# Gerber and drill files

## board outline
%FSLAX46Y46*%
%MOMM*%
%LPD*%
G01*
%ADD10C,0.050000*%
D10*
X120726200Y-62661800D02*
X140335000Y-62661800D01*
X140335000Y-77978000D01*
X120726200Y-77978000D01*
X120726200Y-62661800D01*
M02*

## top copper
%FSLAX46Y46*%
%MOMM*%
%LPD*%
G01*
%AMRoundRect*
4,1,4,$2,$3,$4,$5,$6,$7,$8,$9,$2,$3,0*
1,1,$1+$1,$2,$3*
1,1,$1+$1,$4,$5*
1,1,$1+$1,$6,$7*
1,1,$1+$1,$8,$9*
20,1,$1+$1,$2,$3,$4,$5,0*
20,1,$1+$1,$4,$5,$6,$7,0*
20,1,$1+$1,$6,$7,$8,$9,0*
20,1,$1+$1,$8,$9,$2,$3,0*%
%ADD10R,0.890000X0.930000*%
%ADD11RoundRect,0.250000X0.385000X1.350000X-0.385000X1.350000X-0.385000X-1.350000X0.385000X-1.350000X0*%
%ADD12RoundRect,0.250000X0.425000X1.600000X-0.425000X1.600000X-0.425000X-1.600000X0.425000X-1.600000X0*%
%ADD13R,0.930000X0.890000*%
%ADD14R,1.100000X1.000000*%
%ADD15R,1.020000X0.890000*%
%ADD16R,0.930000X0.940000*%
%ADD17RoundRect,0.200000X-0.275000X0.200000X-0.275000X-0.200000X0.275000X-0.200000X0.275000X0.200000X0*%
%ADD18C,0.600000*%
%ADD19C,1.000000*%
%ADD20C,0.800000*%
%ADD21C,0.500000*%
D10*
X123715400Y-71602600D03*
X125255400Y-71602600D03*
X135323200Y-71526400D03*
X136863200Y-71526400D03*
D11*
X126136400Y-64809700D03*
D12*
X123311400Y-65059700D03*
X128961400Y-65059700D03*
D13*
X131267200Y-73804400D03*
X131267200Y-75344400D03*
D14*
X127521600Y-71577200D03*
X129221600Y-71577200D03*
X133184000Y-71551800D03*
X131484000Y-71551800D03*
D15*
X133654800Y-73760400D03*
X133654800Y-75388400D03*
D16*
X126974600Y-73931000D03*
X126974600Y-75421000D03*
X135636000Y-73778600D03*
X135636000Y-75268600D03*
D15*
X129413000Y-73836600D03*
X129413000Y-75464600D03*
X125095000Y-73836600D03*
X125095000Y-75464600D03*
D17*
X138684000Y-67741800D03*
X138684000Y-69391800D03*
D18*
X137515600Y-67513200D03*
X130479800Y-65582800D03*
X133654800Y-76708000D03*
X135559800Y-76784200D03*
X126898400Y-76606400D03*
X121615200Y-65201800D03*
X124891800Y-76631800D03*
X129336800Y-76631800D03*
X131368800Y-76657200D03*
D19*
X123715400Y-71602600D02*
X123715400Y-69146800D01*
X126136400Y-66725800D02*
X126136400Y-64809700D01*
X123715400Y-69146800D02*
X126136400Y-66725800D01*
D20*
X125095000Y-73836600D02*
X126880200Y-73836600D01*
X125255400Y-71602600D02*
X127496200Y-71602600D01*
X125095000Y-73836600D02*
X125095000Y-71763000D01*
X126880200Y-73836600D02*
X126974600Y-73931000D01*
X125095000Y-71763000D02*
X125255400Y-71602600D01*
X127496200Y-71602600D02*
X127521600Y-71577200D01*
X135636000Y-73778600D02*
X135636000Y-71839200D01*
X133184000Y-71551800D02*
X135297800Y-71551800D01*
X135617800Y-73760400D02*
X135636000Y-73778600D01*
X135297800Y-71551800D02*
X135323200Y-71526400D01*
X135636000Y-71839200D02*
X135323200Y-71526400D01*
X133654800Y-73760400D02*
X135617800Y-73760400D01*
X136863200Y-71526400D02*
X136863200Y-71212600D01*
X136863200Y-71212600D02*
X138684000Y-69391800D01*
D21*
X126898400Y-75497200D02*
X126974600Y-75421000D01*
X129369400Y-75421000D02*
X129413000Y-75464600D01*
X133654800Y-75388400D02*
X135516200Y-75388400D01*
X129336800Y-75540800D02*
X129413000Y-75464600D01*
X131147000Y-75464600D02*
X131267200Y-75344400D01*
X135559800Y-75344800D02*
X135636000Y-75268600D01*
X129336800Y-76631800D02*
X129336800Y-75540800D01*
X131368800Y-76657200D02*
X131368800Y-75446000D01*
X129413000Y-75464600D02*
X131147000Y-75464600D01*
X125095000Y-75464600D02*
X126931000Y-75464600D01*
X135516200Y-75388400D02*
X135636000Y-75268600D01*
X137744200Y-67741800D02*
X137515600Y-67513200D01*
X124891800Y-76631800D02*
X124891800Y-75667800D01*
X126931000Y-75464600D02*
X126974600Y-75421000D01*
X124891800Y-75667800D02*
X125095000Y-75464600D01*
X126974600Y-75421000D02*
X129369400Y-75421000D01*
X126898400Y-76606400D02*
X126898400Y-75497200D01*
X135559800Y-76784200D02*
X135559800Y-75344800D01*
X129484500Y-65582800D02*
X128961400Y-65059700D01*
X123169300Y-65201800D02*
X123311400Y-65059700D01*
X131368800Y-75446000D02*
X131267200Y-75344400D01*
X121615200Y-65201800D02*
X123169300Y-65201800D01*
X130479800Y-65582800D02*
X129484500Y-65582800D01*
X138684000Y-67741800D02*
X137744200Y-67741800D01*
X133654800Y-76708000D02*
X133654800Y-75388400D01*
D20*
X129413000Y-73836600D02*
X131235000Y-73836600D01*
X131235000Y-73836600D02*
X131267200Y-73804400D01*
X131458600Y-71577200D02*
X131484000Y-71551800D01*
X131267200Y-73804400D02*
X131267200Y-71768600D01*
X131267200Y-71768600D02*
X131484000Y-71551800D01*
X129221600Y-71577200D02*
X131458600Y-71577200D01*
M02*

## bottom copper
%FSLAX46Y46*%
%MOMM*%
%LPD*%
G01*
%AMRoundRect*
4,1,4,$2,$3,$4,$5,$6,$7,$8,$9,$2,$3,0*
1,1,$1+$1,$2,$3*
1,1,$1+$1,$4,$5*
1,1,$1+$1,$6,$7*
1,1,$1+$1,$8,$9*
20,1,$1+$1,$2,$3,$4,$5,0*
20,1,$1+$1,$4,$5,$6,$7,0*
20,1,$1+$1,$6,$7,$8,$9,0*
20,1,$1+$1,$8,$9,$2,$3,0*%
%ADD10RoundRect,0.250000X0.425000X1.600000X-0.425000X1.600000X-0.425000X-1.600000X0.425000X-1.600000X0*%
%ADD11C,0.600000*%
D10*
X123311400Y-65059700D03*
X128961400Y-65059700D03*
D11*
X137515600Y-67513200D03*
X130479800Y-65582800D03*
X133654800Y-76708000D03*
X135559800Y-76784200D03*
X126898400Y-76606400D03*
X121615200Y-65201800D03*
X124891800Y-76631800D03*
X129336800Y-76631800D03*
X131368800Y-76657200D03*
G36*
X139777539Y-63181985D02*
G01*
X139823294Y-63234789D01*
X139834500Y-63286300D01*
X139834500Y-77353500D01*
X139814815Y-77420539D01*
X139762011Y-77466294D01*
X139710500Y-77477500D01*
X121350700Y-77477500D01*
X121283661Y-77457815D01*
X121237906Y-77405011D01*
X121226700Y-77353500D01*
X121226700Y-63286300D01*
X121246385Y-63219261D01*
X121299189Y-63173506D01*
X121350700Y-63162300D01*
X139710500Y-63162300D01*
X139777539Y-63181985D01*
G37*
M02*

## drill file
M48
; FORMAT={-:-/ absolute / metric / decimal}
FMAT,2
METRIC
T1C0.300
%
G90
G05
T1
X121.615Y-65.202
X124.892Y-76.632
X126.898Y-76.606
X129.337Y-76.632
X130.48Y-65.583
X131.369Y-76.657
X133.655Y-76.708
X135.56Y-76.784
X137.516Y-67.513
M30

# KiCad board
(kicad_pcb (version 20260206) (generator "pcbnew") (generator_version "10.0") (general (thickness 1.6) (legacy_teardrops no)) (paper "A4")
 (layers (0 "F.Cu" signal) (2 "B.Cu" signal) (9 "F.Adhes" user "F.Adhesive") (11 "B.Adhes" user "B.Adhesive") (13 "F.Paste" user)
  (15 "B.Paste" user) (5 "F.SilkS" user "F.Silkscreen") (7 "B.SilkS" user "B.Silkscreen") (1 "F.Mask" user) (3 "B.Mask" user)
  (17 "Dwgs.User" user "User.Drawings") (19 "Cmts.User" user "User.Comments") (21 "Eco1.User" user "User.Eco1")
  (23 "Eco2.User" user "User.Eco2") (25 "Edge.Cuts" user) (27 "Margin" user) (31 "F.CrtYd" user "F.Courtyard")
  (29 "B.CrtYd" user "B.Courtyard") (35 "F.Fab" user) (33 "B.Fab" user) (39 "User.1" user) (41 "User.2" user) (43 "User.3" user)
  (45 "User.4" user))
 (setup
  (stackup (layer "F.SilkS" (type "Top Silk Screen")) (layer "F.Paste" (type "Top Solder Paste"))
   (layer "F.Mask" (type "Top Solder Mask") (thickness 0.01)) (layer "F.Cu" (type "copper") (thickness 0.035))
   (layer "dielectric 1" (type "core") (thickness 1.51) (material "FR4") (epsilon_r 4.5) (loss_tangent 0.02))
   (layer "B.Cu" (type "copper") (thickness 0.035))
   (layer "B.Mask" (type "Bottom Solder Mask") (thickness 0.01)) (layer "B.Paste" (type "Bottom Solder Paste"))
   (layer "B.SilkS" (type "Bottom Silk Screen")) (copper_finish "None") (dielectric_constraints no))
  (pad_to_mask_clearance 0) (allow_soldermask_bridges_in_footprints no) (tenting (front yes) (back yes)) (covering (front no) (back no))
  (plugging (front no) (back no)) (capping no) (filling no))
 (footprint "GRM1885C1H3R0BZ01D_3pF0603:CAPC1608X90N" (layer "F.Cu") (at 124.4854 71.6026)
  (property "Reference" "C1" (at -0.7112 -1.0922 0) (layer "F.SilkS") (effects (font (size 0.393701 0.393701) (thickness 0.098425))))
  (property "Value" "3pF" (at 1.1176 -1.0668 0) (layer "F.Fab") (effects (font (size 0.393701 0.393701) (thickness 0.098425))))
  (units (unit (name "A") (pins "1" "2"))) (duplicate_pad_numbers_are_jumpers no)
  (pad "1" smd rect (at -0.77 0) (size 0.89 0.93) (layers "F.Cu" "F.Mask" "F.Paste") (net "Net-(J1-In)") (solder_mask_margin 0.102))
  (pad "2" smd rect (at 0.77 0) (size 0.89 0.93) (layers "F.Cu" "F.Mask" "F.Paste") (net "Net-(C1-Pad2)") (solder_mask_margin 0.102)))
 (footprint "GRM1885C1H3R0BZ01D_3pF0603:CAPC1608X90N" (layer "F.Cu") (at 136.0932 71.5264)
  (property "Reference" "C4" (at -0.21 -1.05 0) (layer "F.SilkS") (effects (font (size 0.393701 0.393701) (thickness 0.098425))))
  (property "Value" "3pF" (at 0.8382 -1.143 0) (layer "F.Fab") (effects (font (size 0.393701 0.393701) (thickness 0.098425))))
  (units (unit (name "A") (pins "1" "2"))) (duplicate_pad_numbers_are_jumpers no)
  (pad "1" smd rect (at -0.77 0) (size 0.89 0.93) (layers "F.Cu" "F.Mask" "F.Paste") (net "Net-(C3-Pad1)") (solder_mask_margin 0.102))
  (pad "2" smd rect (at 0.77 0) (size 0.89 0.93) (layers "F.Cu" "F.Mask" "F.Paste") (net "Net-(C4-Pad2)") (solder_mask_margin 0.102)))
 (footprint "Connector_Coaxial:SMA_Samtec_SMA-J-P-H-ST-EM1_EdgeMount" (layer "F.Cu") (at 126.1364 64.8097 90)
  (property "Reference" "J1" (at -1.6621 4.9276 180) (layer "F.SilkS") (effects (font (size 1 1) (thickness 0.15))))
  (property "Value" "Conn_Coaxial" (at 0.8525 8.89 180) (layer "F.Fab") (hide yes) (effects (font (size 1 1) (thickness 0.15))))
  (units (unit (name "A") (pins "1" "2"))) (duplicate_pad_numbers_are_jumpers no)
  (pad "1" smd roundrect (at 0 0 180) (size 1.27 3.2) (layers "F.Cu" "F.Mask") (roundrect_rratio 0.1968503937) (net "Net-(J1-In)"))
  (pad "2" smd roundrect (at -0.25 -2.825 180) (size 1.35 3.7) (layers "F.Cu" "F.Mask") (roundrect_rratio 0.1851851852) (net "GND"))
  (pad "2" smd roundrect (at -0.25 -2.825 180) (size 1.35 3.7) (layers "B.Cu" "B.Mask") (roundrect_rratio 0.1851851852) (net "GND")
   (zone_connect 2))
  (pad "2" smd roundrect (at -0.25 2.825 180) (size 1.35 3.7) (layers "F.Cu" "F.Mask") (roundrect_rratio 0.1851851852) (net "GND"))
  (pad "2" smd roundrect (at -0.25 2.825 180) (size 1.35 3.7) (layers "B.Cu" "B.Mask") (roundrect_rratio 0.1851851852) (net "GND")
   (zone_connect 2)))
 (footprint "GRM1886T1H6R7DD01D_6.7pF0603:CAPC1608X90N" (layer "F.Cu") (at 131.2672 74.5744 -90)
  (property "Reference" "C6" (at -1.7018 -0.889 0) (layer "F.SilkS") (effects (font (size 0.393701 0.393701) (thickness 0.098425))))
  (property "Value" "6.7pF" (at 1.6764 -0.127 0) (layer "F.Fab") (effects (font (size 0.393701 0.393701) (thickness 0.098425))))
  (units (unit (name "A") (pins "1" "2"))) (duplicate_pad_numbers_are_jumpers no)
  (pad "1" smd rect (at -0.77 0 270) (size 0.89 0.93) (layers "F.Cu" "F.Mask" "F.Paste") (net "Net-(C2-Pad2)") (solder_mask_margin 0.102))
  (pad "2" smd rect (at 0.77 0 270) (size 0.89 0.93) (layers "F.Cu" "F.Mask" "F.Paste") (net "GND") (solder_mask_margin 0.102)))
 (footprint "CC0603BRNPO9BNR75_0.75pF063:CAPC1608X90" (layer "F.Cu") (at 128.3716 71.5772)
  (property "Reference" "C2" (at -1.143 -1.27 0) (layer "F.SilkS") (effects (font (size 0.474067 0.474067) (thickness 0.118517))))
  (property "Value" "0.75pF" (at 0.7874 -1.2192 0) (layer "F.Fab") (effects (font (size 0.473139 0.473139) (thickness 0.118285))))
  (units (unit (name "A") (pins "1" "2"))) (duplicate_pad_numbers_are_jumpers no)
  (pad "1" smd rect (at -0.85 0) (size 1.1 1) (layers "F.Cu" "F.Mask" "F.Paste") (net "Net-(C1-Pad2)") (solder_mask_margin 0.102))
  (pad "2" smd rect (at 0.85 0) (size 1.1 1) (layers "F.Cu" "F.Mask" "F.Paste") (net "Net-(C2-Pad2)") (solder_mask_margin 0.102)))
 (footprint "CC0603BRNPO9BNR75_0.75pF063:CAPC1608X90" (layer "F.Cu") (at 132.334 71.5518 180)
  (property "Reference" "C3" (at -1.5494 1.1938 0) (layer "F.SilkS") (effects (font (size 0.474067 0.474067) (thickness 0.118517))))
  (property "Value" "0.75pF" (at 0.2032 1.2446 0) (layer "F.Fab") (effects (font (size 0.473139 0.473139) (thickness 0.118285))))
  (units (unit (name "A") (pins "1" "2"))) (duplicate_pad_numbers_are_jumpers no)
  (pad "1" smd rect (at -0.85 0 180) (size 1.1 1) (layers "F.Cu" "F.Mask" "F.Paste") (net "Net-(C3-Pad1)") (solder_mask_margin 0.102))
  (pad "2" smd rect (at 0.85 0 180) (size 1.1 1) (layers "F.Cu" "F.Mask" "F.Paste") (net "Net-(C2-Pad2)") (solder_mask_margin 0.102)))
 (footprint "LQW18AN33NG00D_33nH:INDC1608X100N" (layer "F.Cu") (at 133.6548 74.5744 -90)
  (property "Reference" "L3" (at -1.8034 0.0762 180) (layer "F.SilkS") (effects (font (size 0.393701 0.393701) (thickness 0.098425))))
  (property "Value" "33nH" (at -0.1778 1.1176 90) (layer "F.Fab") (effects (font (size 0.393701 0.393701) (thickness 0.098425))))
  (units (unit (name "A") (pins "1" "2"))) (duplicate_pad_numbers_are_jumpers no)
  (pad "1" smd rect (at -0.814 0 270) (size 0.89 1.02) (layers "F.Cu" "F.Mask" "F.Paste") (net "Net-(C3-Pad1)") (solder_mask_margin 0.102))
  (pad "2" smd rect (at 0.814 0 270) (size 0.89 1.02) (layers "F.Cu" "F.Mask" "F.Paste") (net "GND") (solder_mask_margin 0.102)))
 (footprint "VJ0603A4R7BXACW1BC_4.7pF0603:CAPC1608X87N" (layer "F.Cu") (at 126.9746 74.676 -90)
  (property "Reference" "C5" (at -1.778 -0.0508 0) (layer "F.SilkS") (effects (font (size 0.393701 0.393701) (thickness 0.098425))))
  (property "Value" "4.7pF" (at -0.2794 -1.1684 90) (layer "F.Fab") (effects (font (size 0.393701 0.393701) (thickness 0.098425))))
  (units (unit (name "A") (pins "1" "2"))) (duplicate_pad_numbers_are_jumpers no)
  (pad "1" smd rect (at -0.745 0 270) (size 0.94 0.93) (layers "F.Cu" "F.Mask" "F.Paste") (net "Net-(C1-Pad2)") (solder_mask_margin 0.102))
  (pad "2" smd rect (at 0.745 0 270) (size 0.94 0.93) (layers "F.Cu" "F.Mask" "F.Paste") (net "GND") (solder_mask_margin 0.102)))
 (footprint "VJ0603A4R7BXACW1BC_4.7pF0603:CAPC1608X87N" (layer "F.Cu") (at 135.636 74.5236 -90)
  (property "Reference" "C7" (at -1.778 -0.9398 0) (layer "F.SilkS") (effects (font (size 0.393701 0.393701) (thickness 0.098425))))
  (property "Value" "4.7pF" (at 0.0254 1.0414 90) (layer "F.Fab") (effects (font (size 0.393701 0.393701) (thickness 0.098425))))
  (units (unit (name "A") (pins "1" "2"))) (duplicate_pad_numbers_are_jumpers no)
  (pad "1" smd rect (at -0.745 0 270) (size 0.94 0.93) (layers "F.Cu" "F.Mask" "F.Paste") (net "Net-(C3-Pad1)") (solder_mask_margin 0.102))
  (pad "2" smd rect (at 0.745 0 270) (size 0.94 0.93) (layers "F.Cu" "F.Mask" "F.Paste") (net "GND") (solder_mask_margin 0.102)))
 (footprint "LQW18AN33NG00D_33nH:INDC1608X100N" (layer "F.Cu") (at 129.413 74.6506 -90)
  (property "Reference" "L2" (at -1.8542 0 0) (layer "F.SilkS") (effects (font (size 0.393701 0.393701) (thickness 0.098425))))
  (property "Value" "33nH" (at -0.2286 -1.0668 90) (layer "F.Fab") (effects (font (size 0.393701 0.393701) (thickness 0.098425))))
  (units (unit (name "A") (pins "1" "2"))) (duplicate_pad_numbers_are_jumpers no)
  (pad "1" smd rect (at -0.814 0 270) (size 0.89 1.02) (layers "F.Cu" "F.Mask" "F.Paste") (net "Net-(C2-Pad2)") (solder_mask_margin 0.102))
  (pad "2" smd rect (at 0.814 0 270) (size 0.89 1.02) (layers "F.Cu" "F.Mask" "F.Paste") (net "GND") (solder_mask_margin 0.102)))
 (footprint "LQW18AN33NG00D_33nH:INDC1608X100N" (layer "F.Cu") (at 125.095 74.6506 -90)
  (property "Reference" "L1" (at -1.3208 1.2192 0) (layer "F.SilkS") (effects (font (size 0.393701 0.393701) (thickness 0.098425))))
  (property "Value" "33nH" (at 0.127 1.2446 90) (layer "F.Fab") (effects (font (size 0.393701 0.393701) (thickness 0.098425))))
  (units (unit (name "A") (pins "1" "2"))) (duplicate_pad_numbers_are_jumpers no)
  (pad "1" smd rect (at -0.814 0 270) (size 0.89 1.02) (layers "F.Cu" "F.Mask" "F.Paste") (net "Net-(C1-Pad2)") (solder_mask_margin 0.102))
  (pad "2" smd rect (at 0.814 0 270) (size 0.89 1.02) (layers "F.Cu" "F.Mask" "F.Paste") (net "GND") (solder_mask_margin 0.102)))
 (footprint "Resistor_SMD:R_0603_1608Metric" (layer "F.Cu") (at 138.684 68.5668 -90)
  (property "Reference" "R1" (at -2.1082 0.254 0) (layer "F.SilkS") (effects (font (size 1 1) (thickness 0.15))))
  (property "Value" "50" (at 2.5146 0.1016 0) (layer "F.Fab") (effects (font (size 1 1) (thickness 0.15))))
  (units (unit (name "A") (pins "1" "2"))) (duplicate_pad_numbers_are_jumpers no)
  (pad "1" smd roundrect (at -0.825 0 270) (size 0.8 0.95) (layers "F.Cu" "F.Mask" "F.Paste") (roundrect_rratio 0.25) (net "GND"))
  (pad "2" smd roundrect (at 0.825 0 270) (size 0.8 0.95) (layers "F.Cu" "F.Mask" "F.Paste") (roundrect_rratio 0.25) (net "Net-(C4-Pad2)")))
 (gr_rect (start 120.7262 62.6618) (end 140.335 77.978) (stroke (width 0.05) (type default)) (fill no) (layer "Edge.Cuts"))
 (segment (start 123.7154 71.6026) (end 123.7154 69.1468) (width 1) (layer "F.Cu") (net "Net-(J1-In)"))
 (segment (start 126.1364 66.7258) (end 126.1364 64.8097) (width 1) (layer "F.Cu") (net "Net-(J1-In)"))
 (segment (start 123.7154 69.1468) (end 126.1364 66.7258) (width 1) (layer "F.Cu") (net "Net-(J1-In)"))
 (segment (start 125.095 73.8366) (end 126.8802 73.8366) (width 0.8) (layer "F.Cu") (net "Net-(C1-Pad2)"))
 (segment (start 125.2554 71.6026) (end 127.4962 71.6026) (width 0.8) (layer "F.Cu") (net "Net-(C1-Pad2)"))
 (segment (start 125.095 73.8366) (end 125.095 71.763) (width 0.8) (layer "F.Cu") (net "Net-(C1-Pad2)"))
 (segment (start 126.8802 73.8366) (end 126.9746 73.931) (width 0.8) (layer "F.Cu") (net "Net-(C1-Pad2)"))
 (segment (start 125.095 71.763) (end 125.2554 71.6026) (width 0.8) (layer "F.Cu") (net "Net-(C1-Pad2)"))
 (segment (start 127.4962 71.6026) (end 127.5216 71.5772) (width 0.8) (layer "F.Cu") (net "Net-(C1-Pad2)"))
 (segment (start 135.636 73.7786) (end 135.636 71.8392) (width 0.8) (layer "F.Cu") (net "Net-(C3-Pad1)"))
 (segment (start 133.184 71.5518) (end 135.2978 71.5518) (width 0.8) (layer "F.Cu") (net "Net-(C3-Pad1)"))
 (segment (start 135.6178 73.7604) (end 135.636 73.7786) (width 0.8) (layer "F.Cu") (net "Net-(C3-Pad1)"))
 (segment (start 135.2978 71.5518) (end 135.3232 71.5264) (width 0.8) (layer "F.Cu") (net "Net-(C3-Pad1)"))
 (segment (start 135.636 71.8392) (end 135.3232 71.5264) (width 0.8) (layer "F.Cu") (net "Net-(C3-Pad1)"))
 (segment (start 133.6548 73.7604) (end 135.6178 73.7604) (width 0.8) (layer "F.Cu") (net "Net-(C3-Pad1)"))
 (segment (start 136.8632 71.5264) (end 136.8632 71.2126) (width 0.8) (layer "F.Cu") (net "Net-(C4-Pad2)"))
 (segment (start 136.8632 71.2126) (end 138.684 69.3918) (width 0.8) (layer "F.Cu") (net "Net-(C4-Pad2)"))
 (segment (start 126.8984 75.4972) (end 126.9746 75.421) (width 0.5) (layer "F.Cu") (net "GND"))
 (segment (start 129.3694 75.421) (end 129.413 75.4646) (width 0.5) (layer "F.Cu") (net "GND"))
 (segment (start 133.6548 75.3884) (end 135.5162 75.3884) (width 0.5) (layer "F.Cu") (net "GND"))
 (segment (start 129.3368 75.5408) (end 129.413 75.4646) (width 0.5) (layer "F.Cu") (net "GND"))
 (segment (start 131.147 75.4646) (end 131.2672 75.3444) (width 0.5) (layer "F.Cu") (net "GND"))
 (segment (start 135.5598 75.3448) (end 135.636 75.2686) (width 0.5) (layer "F.Cu") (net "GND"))
 (segment (start 129.3368 76.6318) (end 129.3368 75.5408) (width 0.5) (layer "F.Cu") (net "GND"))
 (segment (start 131.3688 76.6572) (end 131.3688 75.446) (width 0.5) (layer "F.Cu") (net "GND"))
 (segment (start 129.413 75.4646) (end 131.147 75.4646) (width 0.5) (layer "F.Cu") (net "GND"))
 (segment (start 125.095 75.4646) (end 126.931 75.4646) (width 0.5) (layer "F.Cu") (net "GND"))
 (segment (start 135.5162 75.3884) (end 135.636 75.2686) (width 0.5) (layer "F.Cu") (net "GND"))
 (segment (start 137.7442 67.7418) (end 137.5156 67.5132) (width 0.5) (layer "F.Cu") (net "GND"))
 (segment (start 124.8918 76.6318) (end 124.8918 75.6678) (width 0.5) (layer "F.Cu") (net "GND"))
 (segment (start 126.931 75.4646) (end 126.9746 75.421) (width 0.5) (layer "F.Cu") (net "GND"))
 (segment (start 124.8918 75.6678) (end 125.095 75.4646) (width 0.5) (layer "F.Cu") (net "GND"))
 (segment (start 126.9746 75.421) (end 129.3694 75.421) (width 0.5) (layer "F.Cu") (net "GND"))
 (segment (start 126.8984 76.6064) (end 126.8984 75.4972) (width 0.5) (layer "F.Cu") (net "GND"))
 (segment (start 135.5598 76.7842) (end 135.5598 75.3448) (width 0.5) (layer "F.Cu") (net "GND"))
 (segment (start 129.4845 65.5828) (end 128.9614 65.0597) (width 0.5) (layer "F.Cu") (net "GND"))
 (segment (start 123.1693 65.2018) (end 123.3114 65.0597) (width 0.5) (layer "F.Cu") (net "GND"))
 (segment (start 131.3688 75.446) (end 131.2672 75.3444) (width 0.5) (layer "F.Cu") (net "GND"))
 (segment (start 121.6152 65.2018) (end 123.1693 65.2018) (width 0.5) (layer "F.Cu") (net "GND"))
 (segment (start 130.4798 65.5828) (end 129.4845 65.5828) (width 0.5) (layer "F.Cu") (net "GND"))
 (segment (start 138.684 67.7418) (end 137.7442 67.7418) (width 0.5) (layer "F.Cu") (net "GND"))
 (segment (start 133.6548 76.708) (end 133.6548 75.3884) (width 0.5) (layer "F.Cu") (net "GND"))
 (via (at 137.5156 67.5132) (size 0.6) (drill 0.3) (layers "F.Cu" "B.Cu") (free yes) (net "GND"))
 (via (at 130.4798 65.5828) (size 0.6) (drill 0.3) (layers "F.Cu" "B.Cu") (free yes) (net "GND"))
 (via (at 133.6548 76.708) (size 0.6) (drill 0.3) (layers "F.Cu" "B.Cu") (free yes) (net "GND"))
 (via (at 135.5598 76.7842) (size 0.6) (drill 0.3) (layers "F.Cu" "B.Cu") (free yes) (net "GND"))
 (via (at 126.8984 76.6064) (size 0.6) (drill 0.3) (layers "F.Cu" "B.Cu") (free yes) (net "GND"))
 (via (at 121.6152 65.2018) (size 0.6) (drill 0.3) (layers "F.Cu" "B.Cu") (free yes) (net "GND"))
 (via (at 124.8918 76.6318) (size 0.6) (drill 0.3) (layers "F.Cu" "B.Cu") (free yes) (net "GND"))
 (via (at 129.3368 76.6318) (size 0.6) (drill 0.3) (layers "F.Cu" "B.Cu") (free yes) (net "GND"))
 (via (at 131.3688 76.6572) (size 0.6) (drill 0.3) (layers "F.Cu" "B.Cu") (free yes) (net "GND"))
 (segment (start 129.413 73.8366) (end 131.235 73.8366) (width 0.8) (layer "F.Cu") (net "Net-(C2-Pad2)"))
 (segment (start 131.235 73.8366) (end 131.2672 73.8044) (width 0.8) (layer "F.Cu") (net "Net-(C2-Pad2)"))
 (segment (start 131.4586 71.5772) (end 131.484 71.5518) (width 0.8) (layer "F.Cu") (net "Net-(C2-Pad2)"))
 (segment (start 131.2672 73.8044) (end 131.2672 71.7686) (width 0.8) (layer "F.Cu") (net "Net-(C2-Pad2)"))
 (segment (start 131.2672 71.7686) (end 131.484 71.5518) (width 0.8) (layer "F.Cu") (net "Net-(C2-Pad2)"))
 (segment (start 129.2216 71.5772) (end 131.4586 71.5772) (width 0.8) (layer "F.Cu") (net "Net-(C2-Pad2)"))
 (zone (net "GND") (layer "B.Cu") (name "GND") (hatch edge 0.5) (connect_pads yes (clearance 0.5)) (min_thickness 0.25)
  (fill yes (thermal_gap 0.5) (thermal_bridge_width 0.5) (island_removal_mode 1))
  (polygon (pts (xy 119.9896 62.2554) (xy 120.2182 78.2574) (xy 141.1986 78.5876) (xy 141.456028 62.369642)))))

